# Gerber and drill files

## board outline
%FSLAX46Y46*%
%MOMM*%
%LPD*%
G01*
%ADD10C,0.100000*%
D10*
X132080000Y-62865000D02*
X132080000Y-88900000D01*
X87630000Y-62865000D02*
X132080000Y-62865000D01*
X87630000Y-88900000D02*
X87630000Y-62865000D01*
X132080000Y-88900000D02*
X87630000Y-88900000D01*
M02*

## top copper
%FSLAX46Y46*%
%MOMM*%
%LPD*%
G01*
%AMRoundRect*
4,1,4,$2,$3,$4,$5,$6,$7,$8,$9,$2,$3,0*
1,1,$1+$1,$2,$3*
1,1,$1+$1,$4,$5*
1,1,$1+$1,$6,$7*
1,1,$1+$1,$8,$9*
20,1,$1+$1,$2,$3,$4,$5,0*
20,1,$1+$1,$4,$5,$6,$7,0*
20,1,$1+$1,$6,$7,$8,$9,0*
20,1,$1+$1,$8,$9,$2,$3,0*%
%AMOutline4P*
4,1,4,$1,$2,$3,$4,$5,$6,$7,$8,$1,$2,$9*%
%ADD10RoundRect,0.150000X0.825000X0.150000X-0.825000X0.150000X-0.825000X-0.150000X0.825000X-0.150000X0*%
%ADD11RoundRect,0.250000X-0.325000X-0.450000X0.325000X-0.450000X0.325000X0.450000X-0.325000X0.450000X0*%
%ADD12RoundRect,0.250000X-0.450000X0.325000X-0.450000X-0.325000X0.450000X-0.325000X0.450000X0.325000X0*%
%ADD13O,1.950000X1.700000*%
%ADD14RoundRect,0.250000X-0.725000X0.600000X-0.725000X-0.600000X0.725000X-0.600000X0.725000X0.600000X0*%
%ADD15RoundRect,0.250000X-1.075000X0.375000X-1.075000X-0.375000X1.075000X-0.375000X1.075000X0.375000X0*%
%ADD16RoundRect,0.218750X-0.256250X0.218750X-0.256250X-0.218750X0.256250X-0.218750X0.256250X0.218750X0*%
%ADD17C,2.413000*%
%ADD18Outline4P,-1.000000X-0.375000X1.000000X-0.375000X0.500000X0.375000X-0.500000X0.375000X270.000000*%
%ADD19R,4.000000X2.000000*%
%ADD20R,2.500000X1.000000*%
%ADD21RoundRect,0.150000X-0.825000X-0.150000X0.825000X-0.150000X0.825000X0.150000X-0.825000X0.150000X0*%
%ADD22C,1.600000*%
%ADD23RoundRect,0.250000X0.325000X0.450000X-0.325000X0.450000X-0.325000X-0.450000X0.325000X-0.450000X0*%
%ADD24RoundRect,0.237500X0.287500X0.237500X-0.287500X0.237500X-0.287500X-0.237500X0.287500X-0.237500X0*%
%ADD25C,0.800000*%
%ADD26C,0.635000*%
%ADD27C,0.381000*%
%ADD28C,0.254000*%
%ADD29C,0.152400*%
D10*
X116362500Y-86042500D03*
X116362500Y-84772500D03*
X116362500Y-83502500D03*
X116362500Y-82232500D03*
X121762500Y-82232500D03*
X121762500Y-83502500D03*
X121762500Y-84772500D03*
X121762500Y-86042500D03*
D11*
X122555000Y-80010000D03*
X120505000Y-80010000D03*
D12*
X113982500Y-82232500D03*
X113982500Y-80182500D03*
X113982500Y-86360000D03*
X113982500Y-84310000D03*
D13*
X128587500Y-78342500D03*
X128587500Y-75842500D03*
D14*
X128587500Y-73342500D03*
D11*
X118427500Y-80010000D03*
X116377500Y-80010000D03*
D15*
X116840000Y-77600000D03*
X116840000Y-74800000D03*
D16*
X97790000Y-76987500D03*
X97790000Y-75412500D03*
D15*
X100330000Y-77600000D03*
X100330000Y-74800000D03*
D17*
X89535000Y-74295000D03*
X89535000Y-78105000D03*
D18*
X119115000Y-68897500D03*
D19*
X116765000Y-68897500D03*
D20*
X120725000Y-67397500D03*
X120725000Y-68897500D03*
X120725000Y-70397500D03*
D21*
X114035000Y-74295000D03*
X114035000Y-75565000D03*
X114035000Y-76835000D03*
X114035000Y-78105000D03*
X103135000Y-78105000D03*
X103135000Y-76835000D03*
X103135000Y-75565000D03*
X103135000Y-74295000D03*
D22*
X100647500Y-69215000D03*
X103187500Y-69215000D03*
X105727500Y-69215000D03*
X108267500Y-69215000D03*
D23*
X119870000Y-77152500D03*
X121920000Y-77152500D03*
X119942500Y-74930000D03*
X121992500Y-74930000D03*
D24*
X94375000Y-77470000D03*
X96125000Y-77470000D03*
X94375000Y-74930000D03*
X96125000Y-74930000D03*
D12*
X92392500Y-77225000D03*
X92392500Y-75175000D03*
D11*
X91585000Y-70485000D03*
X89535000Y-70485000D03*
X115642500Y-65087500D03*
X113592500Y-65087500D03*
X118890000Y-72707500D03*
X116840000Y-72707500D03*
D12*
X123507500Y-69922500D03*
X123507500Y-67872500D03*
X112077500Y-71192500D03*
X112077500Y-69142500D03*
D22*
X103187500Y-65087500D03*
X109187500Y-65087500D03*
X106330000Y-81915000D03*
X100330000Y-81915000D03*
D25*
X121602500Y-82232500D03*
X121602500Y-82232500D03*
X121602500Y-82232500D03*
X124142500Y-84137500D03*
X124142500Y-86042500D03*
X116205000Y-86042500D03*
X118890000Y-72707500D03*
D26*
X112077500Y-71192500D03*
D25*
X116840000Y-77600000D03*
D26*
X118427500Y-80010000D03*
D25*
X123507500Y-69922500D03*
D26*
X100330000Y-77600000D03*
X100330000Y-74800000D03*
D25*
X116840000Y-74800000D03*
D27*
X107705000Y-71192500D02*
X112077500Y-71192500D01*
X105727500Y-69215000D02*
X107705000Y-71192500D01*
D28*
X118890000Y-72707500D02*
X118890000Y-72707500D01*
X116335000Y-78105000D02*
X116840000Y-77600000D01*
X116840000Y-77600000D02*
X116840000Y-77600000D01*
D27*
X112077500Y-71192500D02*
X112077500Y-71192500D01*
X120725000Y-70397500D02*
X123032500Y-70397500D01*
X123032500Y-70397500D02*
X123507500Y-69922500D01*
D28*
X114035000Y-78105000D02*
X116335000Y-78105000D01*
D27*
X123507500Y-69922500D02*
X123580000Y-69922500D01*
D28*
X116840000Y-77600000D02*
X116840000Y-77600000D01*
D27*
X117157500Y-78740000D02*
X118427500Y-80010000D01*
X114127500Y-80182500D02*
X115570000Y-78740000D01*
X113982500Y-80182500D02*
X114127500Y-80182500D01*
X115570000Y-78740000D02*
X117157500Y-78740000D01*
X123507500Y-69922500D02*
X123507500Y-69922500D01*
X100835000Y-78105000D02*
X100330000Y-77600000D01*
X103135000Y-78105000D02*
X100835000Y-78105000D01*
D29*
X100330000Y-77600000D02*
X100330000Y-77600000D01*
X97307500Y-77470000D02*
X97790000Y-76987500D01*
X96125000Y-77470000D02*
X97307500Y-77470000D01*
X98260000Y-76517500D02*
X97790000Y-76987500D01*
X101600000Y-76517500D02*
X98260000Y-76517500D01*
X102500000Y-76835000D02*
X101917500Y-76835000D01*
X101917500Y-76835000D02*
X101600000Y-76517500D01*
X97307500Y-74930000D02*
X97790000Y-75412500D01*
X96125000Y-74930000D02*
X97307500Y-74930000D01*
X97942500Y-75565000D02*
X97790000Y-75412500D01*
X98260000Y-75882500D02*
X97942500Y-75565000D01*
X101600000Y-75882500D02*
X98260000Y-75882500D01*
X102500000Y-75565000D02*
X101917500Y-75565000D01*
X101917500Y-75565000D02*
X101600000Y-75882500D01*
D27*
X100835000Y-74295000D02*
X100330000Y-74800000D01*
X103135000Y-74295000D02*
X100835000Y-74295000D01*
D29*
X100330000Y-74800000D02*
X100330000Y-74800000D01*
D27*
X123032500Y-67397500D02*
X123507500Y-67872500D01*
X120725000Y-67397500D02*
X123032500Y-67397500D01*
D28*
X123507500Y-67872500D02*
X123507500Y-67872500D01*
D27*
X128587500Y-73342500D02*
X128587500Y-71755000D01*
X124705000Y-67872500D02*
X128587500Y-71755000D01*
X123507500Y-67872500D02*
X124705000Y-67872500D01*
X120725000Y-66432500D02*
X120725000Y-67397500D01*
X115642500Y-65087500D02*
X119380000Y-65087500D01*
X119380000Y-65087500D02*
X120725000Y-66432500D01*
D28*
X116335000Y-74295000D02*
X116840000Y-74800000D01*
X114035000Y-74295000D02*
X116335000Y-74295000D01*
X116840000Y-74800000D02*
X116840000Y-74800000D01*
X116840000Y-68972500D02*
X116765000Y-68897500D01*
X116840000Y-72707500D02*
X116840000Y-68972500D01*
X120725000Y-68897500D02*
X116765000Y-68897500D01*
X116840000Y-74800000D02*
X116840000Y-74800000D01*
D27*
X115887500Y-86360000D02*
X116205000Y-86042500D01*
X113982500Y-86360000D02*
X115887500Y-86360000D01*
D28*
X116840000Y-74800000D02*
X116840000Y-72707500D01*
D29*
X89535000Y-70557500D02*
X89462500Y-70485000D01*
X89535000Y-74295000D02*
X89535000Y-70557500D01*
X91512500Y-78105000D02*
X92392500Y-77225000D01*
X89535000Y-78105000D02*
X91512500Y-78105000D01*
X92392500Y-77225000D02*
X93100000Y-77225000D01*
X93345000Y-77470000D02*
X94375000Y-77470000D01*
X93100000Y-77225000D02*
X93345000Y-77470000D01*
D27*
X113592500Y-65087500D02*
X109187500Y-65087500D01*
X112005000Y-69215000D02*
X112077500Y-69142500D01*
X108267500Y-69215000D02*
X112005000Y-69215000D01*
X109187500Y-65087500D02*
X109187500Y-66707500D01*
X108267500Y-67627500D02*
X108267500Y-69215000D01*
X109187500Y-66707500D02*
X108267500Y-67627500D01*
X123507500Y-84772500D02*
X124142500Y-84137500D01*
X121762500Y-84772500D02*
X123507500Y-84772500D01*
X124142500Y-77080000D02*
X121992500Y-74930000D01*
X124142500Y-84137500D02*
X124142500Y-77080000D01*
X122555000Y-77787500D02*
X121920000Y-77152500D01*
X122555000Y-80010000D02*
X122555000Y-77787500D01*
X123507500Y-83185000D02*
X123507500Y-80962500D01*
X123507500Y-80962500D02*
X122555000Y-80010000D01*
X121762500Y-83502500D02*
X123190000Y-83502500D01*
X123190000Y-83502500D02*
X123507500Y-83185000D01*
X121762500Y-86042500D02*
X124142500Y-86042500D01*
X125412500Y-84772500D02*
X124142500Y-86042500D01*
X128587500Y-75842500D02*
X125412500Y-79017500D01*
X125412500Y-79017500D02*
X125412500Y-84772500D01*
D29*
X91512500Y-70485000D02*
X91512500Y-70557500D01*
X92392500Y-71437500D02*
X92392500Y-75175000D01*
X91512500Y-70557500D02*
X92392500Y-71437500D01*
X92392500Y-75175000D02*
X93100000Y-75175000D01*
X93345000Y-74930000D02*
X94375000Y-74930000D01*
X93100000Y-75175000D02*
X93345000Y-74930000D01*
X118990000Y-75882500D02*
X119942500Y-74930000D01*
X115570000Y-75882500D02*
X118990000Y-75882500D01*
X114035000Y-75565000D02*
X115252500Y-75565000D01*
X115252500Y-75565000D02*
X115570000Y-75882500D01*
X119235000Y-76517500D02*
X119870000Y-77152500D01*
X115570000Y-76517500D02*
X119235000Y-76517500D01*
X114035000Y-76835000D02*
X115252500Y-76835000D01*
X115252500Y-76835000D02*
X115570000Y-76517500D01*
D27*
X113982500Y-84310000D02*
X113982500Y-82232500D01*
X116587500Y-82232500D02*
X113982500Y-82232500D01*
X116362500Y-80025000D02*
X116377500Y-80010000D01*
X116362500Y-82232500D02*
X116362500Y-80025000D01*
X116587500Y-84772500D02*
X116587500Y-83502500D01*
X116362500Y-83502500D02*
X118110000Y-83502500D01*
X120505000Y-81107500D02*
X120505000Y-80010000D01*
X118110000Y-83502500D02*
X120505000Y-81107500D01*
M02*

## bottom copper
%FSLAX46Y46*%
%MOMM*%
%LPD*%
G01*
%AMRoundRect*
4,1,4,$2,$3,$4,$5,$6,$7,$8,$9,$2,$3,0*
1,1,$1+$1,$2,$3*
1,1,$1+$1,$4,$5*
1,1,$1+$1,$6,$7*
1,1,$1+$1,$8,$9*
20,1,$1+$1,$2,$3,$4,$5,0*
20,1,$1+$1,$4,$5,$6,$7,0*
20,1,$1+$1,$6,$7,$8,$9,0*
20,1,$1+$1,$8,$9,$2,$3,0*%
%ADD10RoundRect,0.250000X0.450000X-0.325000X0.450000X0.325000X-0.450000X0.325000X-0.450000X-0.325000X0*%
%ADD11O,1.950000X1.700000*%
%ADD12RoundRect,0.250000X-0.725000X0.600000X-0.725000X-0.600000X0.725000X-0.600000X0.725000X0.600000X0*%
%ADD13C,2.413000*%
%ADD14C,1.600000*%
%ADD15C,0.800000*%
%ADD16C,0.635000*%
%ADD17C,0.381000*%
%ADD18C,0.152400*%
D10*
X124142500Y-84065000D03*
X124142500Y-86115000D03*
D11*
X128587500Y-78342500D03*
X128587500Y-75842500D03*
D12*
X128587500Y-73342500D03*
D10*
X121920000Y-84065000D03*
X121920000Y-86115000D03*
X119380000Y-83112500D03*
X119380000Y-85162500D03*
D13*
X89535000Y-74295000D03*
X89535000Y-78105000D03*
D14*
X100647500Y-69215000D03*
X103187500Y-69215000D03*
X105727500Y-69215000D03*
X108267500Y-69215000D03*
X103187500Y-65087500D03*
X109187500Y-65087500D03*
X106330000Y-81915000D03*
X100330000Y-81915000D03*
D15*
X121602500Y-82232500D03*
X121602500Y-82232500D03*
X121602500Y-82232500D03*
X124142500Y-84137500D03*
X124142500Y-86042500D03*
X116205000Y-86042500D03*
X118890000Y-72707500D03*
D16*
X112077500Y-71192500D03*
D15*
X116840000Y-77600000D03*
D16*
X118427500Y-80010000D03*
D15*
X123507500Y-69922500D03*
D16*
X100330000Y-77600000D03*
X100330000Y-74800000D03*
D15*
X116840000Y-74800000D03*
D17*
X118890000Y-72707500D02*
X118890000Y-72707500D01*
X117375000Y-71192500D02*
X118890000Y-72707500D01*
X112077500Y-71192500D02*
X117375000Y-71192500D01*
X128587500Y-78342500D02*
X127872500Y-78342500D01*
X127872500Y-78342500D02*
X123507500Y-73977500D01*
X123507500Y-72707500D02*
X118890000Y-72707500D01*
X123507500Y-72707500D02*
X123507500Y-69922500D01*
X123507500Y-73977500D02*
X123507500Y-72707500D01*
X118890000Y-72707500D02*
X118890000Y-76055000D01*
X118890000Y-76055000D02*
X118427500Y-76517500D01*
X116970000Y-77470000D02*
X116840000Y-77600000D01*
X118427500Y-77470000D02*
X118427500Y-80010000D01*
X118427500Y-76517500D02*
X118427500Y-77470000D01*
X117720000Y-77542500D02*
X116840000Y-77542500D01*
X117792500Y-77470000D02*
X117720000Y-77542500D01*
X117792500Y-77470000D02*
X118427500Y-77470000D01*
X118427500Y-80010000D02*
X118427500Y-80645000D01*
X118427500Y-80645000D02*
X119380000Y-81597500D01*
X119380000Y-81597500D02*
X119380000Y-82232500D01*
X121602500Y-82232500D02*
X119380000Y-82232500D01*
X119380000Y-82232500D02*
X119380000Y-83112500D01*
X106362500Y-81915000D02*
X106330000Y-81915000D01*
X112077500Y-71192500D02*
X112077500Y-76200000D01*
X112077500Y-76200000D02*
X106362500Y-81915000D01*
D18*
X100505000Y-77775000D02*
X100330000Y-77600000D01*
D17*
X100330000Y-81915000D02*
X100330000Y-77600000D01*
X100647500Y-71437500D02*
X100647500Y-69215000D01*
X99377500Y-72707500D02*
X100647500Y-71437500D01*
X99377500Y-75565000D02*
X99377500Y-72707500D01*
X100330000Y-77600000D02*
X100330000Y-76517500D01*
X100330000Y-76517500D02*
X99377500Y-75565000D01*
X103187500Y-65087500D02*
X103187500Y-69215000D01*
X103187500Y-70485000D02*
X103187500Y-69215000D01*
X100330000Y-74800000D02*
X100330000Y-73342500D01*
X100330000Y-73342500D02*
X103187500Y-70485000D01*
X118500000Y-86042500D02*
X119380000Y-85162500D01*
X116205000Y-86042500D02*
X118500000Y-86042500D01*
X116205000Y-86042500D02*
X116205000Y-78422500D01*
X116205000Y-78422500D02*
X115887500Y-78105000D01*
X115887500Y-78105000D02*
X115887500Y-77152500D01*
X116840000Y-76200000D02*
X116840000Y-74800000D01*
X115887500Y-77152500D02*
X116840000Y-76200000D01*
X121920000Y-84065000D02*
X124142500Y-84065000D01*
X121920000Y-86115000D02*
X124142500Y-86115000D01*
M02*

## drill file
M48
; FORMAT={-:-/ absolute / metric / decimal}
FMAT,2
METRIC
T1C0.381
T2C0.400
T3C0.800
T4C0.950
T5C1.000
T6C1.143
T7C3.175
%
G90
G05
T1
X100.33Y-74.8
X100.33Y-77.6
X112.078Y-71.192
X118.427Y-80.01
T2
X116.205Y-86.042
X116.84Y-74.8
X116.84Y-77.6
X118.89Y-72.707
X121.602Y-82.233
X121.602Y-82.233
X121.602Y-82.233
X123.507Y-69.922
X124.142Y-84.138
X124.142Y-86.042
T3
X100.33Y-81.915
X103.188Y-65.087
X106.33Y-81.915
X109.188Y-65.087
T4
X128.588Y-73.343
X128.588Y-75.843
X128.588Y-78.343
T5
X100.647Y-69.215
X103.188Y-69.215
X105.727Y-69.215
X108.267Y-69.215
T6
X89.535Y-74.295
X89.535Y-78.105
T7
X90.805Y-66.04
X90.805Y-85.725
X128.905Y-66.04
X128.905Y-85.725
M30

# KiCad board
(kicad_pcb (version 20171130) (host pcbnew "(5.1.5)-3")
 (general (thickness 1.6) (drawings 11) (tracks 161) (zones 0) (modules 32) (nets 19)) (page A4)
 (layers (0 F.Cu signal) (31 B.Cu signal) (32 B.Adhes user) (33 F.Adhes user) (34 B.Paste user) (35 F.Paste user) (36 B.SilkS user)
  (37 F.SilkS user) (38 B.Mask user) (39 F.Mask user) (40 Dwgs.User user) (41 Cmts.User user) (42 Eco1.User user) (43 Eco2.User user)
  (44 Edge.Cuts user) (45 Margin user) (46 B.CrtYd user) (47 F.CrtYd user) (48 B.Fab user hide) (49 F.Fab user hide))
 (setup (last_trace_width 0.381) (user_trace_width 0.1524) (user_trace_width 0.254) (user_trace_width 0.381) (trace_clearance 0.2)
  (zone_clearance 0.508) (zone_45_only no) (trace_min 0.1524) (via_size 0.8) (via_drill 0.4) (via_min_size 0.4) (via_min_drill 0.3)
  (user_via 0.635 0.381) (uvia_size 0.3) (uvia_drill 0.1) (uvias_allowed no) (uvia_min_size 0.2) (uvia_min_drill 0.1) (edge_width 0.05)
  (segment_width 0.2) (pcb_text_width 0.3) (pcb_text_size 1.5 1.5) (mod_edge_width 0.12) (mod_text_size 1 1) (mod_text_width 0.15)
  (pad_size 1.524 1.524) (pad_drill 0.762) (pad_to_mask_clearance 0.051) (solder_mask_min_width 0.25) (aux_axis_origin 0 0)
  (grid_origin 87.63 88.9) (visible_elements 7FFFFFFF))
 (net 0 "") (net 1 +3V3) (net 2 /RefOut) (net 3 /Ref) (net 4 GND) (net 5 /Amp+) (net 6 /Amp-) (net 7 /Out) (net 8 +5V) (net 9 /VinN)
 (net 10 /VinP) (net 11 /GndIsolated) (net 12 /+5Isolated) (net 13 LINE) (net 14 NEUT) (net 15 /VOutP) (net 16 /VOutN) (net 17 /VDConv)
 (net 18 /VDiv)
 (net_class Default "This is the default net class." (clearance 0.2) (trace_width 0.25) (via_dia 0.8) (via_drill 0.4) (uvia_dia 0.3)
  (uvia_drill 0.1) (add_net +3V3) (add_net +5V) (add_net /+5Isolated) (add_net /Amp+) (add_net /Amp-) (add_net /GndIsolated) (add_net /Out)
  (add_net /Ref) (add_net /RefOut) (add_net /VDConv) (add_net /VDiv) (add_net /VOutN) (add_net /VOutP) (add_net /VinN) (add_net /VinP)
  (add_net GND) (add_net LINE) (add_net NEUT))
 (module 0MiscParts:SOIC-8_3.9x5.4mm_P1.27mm (layer F.Cu) (at 119.0625 84.1375 180)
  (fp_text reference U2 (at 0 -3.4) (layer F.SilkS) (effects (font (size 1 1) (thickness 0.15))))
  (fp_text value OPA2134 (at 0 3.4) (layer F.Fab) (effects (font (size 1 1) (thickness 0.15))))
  (pad 8 smd roundrect (at 2.7 -1.905 180) (size 1.95 0.6) (layers F.Cu F.Paste F.Mask) (roundrect_rratio 0.25) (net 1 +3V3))
  (pad 7 smd roundrect (at 2.7 -0.635 180) (size 1.95 0.6) (layers F.Cu F.Paste F.Mask) (roundrect_rratio 0.25) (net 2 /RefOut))
  (pad 6 smd roundrect (at 2.7 0.635 180) (size 1.95 0.6) (layers F.Cu F.Paste F.Mask) (roundrect_rratio 0.25) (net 2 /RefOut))
  (pad 5 smd roundrect (at 2.7 1.905 180) (size 1.95 0.6) (layers F.Cu F.Paste F.Mask) (roundrect_rratio 0.25) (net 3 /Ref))
  (pad 4 smd roundrect (at -2.7 1.905 180) (size 1.95 0.6) (layers F.Cu F.Paste F.Mask) (roundrect_rratio 0.25) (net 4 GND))
  (pad 3 smd roundrect (at -2.7 0.635 180) (size 1.95 0.6) (layers F.Cu F.Paste F.Mask) (roundrect_rratio 0.25) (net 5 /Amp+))
  (pad 2 smd roundrect (at -2.7 -0.635 180) (size 1.95 0.6) (layers F.Cu F.Paste F.Mask) (roundrect_rratio 0.25) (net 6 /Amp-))
  (pad 1 smd roundrect (at -2.7 -1.905 180) (size 1.95 0.6) (layers F.Cu F.Paste F.Mask) (roundrect_rratio 0.25) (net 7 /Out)))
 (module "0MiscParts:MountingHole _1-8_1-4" (layer F.Cu) (at 128.905 85.725)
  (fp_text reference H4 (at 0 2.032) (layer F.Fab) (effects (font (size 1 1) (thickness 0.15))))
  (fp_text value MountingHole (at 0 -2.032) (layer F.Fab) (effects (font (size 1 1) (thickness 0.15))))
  (pad "" np_thru_hole circle (at 0 0) (size 3.175 3.175) (drill 3.175) (layers *.Cu *.Mask)))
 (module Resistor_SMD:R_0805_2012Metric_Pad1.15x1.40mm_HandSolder (layer B.Cu) (at 124.1425 85.09 90)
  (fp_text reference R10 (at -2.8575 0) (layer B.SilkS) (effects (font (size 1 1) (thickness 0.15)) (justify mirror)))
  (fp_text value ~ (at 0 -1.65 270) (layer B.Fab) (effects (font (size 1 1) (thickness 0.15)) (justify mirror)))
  (pad 2 smd roundrect (at 1.025 0 90) (size 1.15 1.4) (layers B.Cu B.Paste B.Mask) (roundrect_rratio 0.217391) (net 6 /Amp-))
  (pad 1 smd roundrect (at -1.025 0 90) (size 1.15 1.4) (layers B.Cu B.Paste B.Mask) (roundrect_rratio 0.217391) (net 7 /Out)))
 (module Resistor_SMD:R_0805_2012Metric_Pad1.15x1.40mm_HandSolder (layer F.Cu) (at 121.53 80.01)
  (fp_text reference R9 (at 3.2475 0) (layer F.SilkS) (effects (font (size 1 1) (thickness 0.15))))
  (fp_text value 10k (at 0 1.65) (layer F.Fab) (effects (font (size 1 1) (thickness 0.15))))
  (pad 2 smd roundrect (at 1.025 0) (size 1.15 1.4) (layers F.Cu F.Paste F.Mask) (roundrect_rratio 0.217391) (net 5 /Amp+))
  (pad 1 smd roundrect (at -1.025 0) (size 1.15 1.4) (layers F.Cu F.Paste F.Mask) (roundrect_rratio 0.217391) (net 2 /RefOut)))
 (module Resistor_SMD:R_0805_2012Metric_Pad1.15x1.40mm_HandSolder (layer F.Cu) (at 113.9825 81.2075 270)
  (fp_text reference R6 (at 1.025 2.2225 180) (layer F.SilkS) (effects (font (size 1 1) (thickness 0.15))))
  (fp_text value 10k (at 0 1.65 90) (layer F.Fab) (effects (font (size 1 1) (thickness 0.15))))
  (pad 2 smd roundrect (at 1.025 0 270) (size 1.15 1.4) (layers F.Cu F.Paste F.Mask) (roundrect_rratio 0.217391) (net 3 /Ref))
  (pad 1 smd roundrect (at -1.025 0 270) (size 1.15 1.4) (layers F.Cu F.Paste F.Mask) (roundrect_rratio 0.217391) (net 4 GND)))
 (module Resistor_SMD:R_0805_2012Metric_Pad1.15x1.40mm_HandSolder (layer F.Cu) (at 113.9825 85.335 270)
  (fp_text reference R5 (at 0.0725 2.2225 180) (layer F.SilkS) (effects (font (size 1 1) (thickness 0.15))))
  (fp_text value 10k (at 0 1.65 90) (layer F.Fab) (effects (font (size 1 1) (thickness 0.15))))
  (pad 2 smd roundrect (at 1.025 0 270) (size 1.15 1.4) (layers F.Cu F.Paste F.Mask) (roundrect_rratio 0.217391) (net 1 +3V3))
  (pad 1 smd roundrect (at -1.025 0 270) (size 1.15 1.4) (layers F.Cu F.Paste F.Mask) (roundrect_rratio 0.217391) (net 3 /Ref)))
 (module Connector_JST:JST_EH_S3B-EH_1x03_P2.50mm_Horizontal (layer F.Cu) (at 128.5875 73.3425 270)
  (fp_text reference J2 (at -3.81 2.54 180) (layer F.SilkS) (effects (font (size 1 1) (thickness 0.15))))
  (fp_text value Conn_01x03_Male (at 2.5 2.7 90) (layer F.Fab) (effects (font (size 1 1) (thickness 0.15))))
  (pad 3 thru_hole oval (at 5 0 270) (size 1.7 1.95) (drill 0.95) (layers *.Cu *.Mask) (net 4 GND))
  (pad 2 thru_hole oval (at 2.5 0 270) (size 1.7 1.95) (drill 0.95) (layers *.Cu *.Mask) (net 7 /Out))
  (pad 1 thru_hole roundrect (at 0 0 270) (size 1.7 1.95) (drill 0.95) (layers *.Cu *.Mask) (roundrect_rratio 0.147059) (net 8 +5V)))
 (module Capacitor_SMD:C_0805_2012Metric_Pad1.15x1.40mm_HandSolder (layer B.Cu) (at 121.92 85.09 90)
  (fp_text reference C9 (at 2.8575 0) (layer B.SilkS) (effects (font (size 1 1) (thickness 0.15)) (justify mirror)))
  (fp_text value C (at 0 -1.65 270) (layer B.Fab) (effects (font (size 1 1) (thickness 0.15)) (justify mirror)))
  (pad 2 smd roundrect (at 1.025 0 90) (size 1.15 1.4) (layers B.Cu B.Paste B.Mask) (roundrect_rratio 0.217391) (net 6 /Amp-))
  (pad 1 smd roundrect (at -1.025 0 90) (size 1.15 1.4) (layers B.Cu B.Paste B.Mask) (roundrect_rratio 0.217391) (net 7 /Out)))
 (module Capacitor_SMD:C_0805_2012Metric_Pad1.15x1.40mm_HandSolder (layer B.Cu) (at 119.38 84.1375 90)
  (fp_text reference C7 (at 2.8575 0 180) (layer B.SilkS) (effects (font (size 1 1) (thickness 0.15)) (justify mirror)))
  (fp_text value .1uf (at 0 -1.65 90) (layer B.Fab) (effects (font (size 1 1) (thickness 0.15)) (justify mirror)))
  (pad 2 smd roundrect (at 1.025 0 90) (size 1.15 1.4) (layers B.Cu B.Paste B.Mask) (roundrect_rratio 0.217391) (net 4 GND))
  (pad 1 smd roundrect (at -1.025 0 90) (size 1.15 1.4) (layers B.Cu B.Paste B.Mask) (roundrect_rratio 0.217391) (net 1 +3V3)))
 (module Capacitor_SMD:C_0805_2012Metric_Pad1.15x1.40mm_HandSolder (layer F.Cu) (at 117.4025 80.01)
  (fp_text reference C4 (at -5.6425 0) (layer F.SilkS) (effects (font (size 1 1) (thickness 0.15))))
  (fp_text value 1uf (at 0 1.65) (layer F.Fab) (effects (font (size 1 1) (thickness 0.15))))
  (pad 2 smd roundrect (at 1.025 0) (size 1.15 1.4) (layers F.Cu F.Paste F.Mask) (roundrect_rratio 0.217391) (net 4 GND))
  (pad 1 smd roundrect (at -1.025 0) (size 1.15 1.4) (layers F.Cu F.Paste F.Mask) (roundrect_rratio 0.217391) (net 3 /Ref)))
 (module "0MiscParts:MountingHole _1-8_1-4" (layer F.Cu) (at 128.905 66.04)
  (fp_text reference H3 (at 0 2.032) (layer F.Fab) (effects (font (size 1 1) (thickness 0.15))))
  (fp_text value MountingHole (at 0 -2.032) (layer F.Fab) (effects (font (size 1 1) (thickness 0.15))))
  (pad "" np_thru_hole circle (at 0 0) (size 3.175 3.175) (drill 3.175) (layers *.Cu *.Mask)))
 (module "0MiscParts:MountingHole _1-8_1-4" (layer F.Cu) (at 90.805 85.725)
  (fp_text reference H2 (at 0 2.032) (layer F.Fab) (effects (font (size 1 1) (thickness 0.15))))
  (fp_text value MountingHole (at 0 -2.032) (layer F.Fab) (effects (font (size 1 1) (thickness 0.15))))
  (pad "" np_thru_hole circle (at 0 0) (size 3.175 3.175) (drill 3.175) (layers *.Cu *.Mask)))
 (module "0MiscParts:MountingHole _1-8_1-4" (layer F.Cu) (at 90.805 66.04)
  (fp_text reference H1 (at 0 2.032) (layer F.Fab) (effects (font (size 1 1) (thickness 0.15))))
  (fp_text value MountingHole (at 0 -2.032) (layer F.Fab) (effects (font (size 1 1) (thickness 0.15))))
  (pad "" np_thru_hole circle (at 0 0) (size 3.175 3.175) (drill 3.175) (layers *.Cu *.Mask)))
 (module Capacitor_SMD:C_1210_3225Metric (layer F.Cu) (at 116.84 76.2 270)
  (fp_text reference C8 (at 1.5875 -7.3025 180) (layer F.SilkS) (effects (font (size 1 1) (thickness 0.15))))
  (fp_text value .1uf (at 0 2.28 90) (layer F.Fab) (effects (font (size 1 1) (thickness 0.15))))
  (pad 2 smd roundrect (at 1.4 0 270) (size 1.25 2.65) (layers F.Cu F.Paste F.Mask) (roundrect_rratio 0.2) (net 4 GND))
  (pad 1 smd roundrect (at -1.4 0 270) (size 1.25 2.65) (layers F.Cu F.Paste F.Mask) (roundrect_rratio 0.2) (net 1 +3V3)))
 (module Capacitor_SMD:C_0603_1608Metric (layer F.Cu) (at 97.79 76.2 270)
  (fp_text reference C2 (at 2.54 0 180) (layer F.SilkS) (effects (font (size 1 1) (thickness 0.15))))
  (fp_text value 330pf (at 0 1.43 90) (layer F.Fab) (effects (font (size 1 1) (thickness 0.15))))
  (pad 2 smd roundrect (at 0.7875 0 270) (size 0.875 0.95) (layers F.Cu F.Paste F.Mask) (roundrect_rratio 0.25) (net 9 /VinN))
  (pad 1 smd roundrect (at -0.7875 0 270) (size 0.875 0.95) (layers F.Cu F.Paste F.Mask) (roundrect_rratio 0.25) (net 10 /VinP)))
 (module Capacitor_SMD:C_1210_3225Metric (layer F.Cu) (at 100.33 76.2 270)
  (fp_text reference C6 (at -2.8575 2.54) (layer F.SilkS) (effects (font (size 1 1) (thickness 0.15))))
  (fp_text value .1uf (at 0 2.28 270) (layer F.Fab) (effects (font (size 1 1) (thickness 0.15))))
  (pad 2 smd roundrect (at 1.4 0 270) (size 1.25 2.65) (layers F.Cu F.Paste F.Mask) (roundrect_rratio 0.2) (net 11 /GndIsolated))
  (pad 1 smd roundrect (at -1.4 0 270) (size 1.25 2.65) (layers F.Cu F.Paste F.Mask) (roundrect_rratio 0.2) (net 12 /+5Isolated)))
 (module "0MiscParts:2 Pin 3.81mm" (layer F.Cu) (at 89.535 76.2 270)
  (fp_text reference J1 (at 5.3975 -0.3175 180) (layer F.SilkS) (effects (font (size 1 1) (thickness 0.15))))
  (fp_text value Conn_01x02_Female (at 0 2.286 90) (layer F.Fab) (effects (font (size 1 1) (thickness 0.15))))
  (pad 1 thru_hole circle (at -1.905 0 270) (size 2.413 2.413) (drill 1.143) (layers *.Cu *.Mask) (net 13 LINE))
  (pad 2 thru_hole circle (at 1.905 0 270) (size 2.413 2.413) (drill 1.143) (layers *.Cu *.Mask) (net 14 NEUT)))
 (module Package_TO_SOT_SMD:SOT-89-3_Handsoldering (layer F.Cu) (at 118.745 68.8975 180)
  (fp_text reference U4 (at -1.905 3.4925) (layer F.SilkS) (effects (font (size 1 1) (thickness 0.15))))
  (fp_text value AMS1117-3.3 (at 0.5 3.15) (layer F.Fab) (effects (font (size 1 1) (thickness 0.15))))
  (pad 2 smd trapezoid (at -0.37 0 270) (size 1.5 0.75) (rect_delta 0 0.5) (layers F.Cu F.Paste F.Mask) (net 1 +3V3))
  (pad 2 smd rect (at 1.98 0 90) (size 2 4) (layers F.Cu F.Paste F.Mask) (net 1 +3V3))
  (pad 3 smd rect (at -1.98 1.5 90) (size 1 2.5) (layers F.Cu F.Paste F.Mask) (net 8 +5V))
  (pad 2 smd rect (at -1.98 0 90) (size 1 2.5) (layers F.Cu F.Paste F.Mask) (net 1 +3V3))
  (pad 1 smd rect (at -1.98 -1.5 90) (size 1 2.5) (layers F.Cu F.Paste F.Mask) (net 4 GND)))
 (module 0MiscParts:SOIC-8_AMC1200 (layer F.Cu) (at 108.585 76.2)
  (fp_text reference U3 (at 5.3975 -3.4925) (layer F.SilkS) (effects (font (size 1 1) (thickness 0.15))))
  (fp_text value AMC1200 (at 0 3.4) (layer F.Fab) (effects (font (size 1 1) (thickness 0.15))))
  (pad 8 smd roundrect (at 5.45 -1.905) (size 1.95 0.6) (layers F.Cu F.Paste F.Mask) (roundrect_rratio 0.25) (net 1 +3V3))
  (pad 7 smd roundrect (at 5.45 -0.635) (size 1.95 0.6) (layers F.Cu F.Paste F.Mask) (roundrect_rratio 0.25) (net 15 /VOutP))
  (pad 6 smd roundrect (at 5.45 0.635) (size 1.95 0.6) (layers F.Cu F.Paste F.Mask) (roundrect_rratio 0.25) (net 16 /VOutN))
  (pad 5 smd roundrect (at 5.45 1.905) (size 1.95 0.6) (layers F.Cu F.Paste F.Mask) (roundrect_rratio 0.25) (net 4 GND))
  (pad 4 smd roundrect (at -5.45 1.905) (size 1.95 0.6) (layers F.Cu F.Paste F.Mask) (roundrect_rratio 0.25) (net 11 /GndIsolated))
  (pad 3 smd roundrect (at -5.45 0.635) (size 1.95 0.6) (layers F.Cu F.Paste F.Mask) (roundrect_rratio 0.25) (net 9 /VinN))
  (pad 2 smd roundrect (at -5.45 -0.635) (size 1.95 0.6) (layers F.Cu F.Paste F.Mask) (roundrect_rratio 0.25) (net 10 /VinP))
  (pad 1 smd roundrect (at -5.45 -1.905) (size 1.95 0.6) (layers F.Cu F.Paste F.Mask) (roundrect_rratio 0.25) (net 12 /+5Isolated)))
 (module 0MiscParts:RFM (layer F.Cu) (at 104.4575 69.215 180)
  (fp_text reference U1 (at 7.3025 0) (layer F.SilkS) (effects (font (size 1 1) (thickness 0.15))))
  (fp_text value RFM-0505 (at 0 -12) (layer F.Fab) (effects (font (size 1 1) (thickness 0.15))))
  (pad 4 thru_hole circle (at 3.81 0 180) (size 1.6 1.6) (drill 1) (layers *.Cu *.Mask) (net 11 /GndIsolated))
  (pad 3 thru_hole circle (at 1.27 0 180) (size 1.6 1.6) (drill 1) (layers *.Cu *.Mask) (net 12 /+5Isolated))
  (pad 2 thru_hole circle (at -1.27 0 180) (size 1.6 1.6) (drill 1) (layers *.Cu *.Mask) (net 4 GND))
  (pad 1 thru_hole circle (at -3.81 0 180) (size 1.6 1.6) (drill 1) (layers *.Cu *.Mask) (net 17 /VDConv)))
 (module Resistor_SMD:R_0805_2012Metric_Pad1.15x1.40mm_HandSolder (layer F.Cu) (at 120.895 77.1525 180)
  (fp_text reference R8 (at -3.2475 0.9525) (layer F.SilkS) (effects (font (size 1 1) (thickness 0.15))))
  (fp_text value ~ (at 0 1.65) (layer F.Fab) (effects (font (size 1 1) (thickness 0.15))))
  (pad 2 smd roundrect (at 1.025 0 180) (size 1.15 1.4) (layers F.Cu F.Paste F.Mask) (roundrect_rratio 0.217391) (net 16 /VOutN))
  (pad 1 smd roundrect (at -1.025 0 180) (size 1.15 1.4) (layers F.Cu F.Paste F.Mask) (roundrect_rratio 0.217391) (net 5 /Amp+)))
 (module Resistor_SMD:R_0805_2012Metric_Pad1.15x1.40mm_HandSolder (layer F.Cu) (at 120.9675 74.93 180)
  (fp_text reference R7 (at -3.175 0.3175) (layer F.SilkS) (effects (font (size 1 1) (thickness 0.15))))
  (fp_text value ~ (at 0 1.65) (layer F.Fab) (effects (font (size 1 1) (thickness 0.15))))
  (pad 2 smd roundrect (at 1.025 0 180) (size 1.15 1.4) (layers F.Cu F.Paste F.Mask) (roundrect_rratio 0.217391) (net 15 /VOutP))
  (pad 1 smd roundrect (at -1.025 0 180) (size 1.15 1.4) (layers F.Cu F.Paste F.Mask) (roundrect_rratio 0.217391) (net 6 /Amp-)))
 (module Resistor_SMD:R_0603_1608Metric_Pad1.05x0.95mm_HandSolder (layer F.Cu) (at 95.25 77.47 180)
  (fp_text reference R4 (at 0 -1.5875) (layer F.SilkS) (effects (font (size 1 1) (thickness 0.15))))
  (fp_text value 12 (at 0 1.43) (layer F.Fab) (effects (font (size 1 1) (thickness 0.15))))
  (pad 2 smd roundrect (at 0.875 0 180) (size 1.05 0.95) (layers F.Cu F.Paste F.Mask) (roundrect_rratio 0.25) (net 14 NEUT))
  (pad 1 smd roundrect (at -0.875 0 180) (size 1.05 0.95) (layers F.Cu F.Paste F.Mask) (roundrect_rratio 0.25) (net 9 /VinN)))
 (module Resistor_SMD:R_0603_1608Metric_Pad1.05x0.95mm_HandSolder (layer F.Cu) (at 95.25 74.93 180)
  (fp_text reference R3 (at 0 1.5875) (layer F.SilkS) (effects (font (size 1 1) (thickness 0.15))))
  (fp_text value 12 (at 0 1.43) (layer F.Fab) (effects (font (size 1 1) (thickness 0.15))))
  (pad 2 smd roundrect (at 0.875 0 180) (size 1.05 0.95) (layers F.Cu F.Paste F.Mask) (roundrect_rratio 0.25) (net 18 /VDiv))
  (pad 1 smd roundrect (at -0.875 0 180) (size 1.05 0.95) (layers F.Cu F.Paste F.Mask) (roundrect_rratio 0.25) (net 10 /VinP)))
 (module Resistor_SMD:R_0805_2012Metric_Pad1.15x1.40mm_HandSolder (layer F.Cu) (at 92.3925 76.2 270)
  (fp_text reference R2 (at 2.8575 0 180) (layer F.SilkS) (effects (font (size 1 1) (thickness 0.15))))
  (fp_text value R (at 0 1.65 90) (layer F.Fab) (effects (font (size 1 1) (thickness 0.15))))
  (pad 2 smd roundrect (at 1.025 0 270) (size 1.15 1.4) (layers F.Cu F.Paste F.Mask) (roundrect_rratio 0.217391) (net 14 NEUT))
  (pad 1 smd roundrect (at -1.025 0 270) (size 1.15 1.4) (layers F.Cu F.Paste F.Mask) (roundrect_rratio 0.217391) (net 18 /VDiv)))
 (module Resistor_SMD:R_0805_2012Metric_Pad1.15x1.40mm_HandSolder (layer F.Cu) (at 90.56 70.485)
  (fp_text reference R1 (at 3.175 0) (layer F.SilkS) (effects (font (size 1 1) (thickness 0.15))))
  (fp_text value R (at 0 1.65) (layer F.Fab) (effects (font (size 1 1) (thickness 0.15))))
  (pad 2 smd roundrect (at 1.025 0) (size 1.15 1.4) (layers F.Cu F.Paste F.Mask) (roundrect_rratio 0.217391) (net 18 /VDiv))
  (pad 1 smd roundrect (at -1.025 0) (size 1.15 1.4) (layers F.Cu F.Paste F.Mask) (roundrect_rratio 0.217391) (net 13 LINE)))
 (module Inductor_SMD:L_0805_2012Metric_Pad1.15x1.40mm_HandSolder (layer F.Cu) (at 114.6175 65.0875)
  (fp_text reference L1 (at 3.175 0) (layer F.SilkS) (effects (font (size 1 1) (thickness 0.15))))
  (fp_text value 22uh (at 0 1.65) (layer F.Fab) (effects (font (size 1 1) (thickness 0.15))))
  (pad 2 smd roundrect (at 1.025 0) (size 1.15 1.4) (layers F.Cu F.Paste F.Mask) (roundrect_rratio 0.217391) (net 8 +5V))
  (pad 1 smd roundrect (at -1.025 0) (size 1.15 1.4) (layers F.Cu F.Paste F.Mask) (roundrect_rratio 0.217391) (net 17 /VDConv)))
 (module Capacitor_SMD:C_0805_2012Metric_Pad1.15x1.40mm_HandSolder (layer F.Cu) (at 117.865 72.7075)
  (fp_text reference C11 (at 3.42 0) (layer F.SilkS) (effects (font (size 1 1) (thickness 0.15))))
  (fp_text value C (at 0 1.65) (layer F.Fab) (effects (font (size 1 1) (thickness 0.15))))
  (pad 2 smd roundrect (at 1.025 0) (size 1.15 1.4) (layers F.Cu F.Paste F.Mask) (roundrect_rratio 0.217391) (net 4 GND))
  (pad 1 smd roundrect (at -1.025 0) (size 1.15 1.4) (layers F.Cu F.Paste F.Mask) (roundrect_rratio 0.217391) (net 1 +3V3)))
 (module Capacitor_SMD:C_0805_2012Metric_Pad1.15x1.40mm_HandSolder (layer F.Cu) (at 123.5075 68.8975 270)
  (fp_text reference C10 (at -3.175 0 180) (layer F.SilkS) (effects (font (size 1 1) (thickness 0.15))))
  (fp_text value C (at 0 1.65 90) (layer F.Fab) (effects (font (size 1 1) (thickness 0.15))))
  (pad 2 smd roundrect (at 1.025 0 270) (size 1.15 1.4) (layers F.Cu F.Paste F.Mask) (roundrect_rratio 0.217391) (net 4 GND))
  (pad 1 smd roundrect (at -1.025 0 270) (size 1.15 1.4) (layers F.Cu F.Paste F.Mask) (roundrect_rratio 0.217391) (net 8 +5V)))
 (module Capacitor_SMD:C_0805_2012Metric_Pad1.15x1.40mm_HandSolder (layer F.Cu) (at 112.0775 70.1675 270)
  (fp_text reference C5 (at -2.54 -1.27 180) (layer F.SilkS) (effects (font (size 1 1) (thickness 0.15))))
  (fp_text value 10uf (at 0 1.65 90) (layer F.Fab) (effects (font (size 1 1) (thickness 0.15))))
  (pad 2 smd roundrect (at 1.025 0 270) (size 1.15 1.4) (layers F.Cu F.Paste F.Mask) (roundrect_rratio 0.217391) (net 4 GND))
  (pad 1 smd roundrect (at -1.025 0 270) (size 1.15 1.4) (layers F.Cu F.Paste F.Mask) (roundrect_rratio 0.217391) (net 17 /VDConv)))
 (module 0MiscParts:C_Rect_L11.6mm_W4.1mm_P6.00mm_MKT (layer F.Cu) (at 106.1875 65.0875 180)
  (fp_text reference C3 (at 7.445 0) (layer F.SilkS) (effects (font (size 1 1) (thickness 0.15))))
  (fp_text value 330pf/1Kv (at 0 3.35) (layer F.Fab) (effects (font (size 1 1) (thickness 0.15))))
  (pad 2 thru_hole circle (at 3 0 180) (size 1.6 1.6) (drill 0.8) (layers *.Cu *.Mask) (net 12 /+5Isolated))
  (pad 1 thru_hole circle (at -3 0 180) (size 1.6 1.6) (drill 0.8) (layers *.Cu *.Mask) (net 17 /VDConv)))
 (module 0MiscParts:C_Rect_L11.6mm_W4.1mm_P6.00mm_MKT (layer F.Cu) (at 103.33 81.915)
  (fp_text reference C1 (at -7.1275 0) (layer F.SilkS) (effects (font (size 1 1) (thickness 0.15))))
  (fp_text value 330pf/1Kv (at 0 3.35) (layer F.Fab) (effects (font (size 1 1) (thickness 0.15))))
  (pad 2 thru_hole circle (at 3 0) (size 1.6 1.6) (drill 0.8) (layers *.Cu *.Mask) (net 4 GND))
  (pad 1 thru_hole circle (at -3 0) (size 1.6 1.6) (drill 0.8) (layers *.Cu *.Mask) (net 11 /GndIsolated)))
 (gr_line (start 132.08 62.865) (end 132.08 88.9) (layer Edge.Cuts) (width 0.1))
 (gr_line (start 87.63 62.865) (end 132.08 62.865) (layer Edge.Cuts) (width 0.1))
 (gr_line (start 87.63 88.9) (end 87.63 62.865) (layer Edge.Cuts) (width 0.1))
 (gr_line (start 132.08 88.9) (end 87.63 88.9) (layer Edge.Cuts) (width 0.1))
 (via (at 121.6025 82.2325) (size 0.8) (drill 0.4) (layers F.Cu B.Cu) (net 4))
 (via (at 121.6025 82.2325) (size 0.8) (drill 0.4) (layers F.Cu B.Cu) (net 4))
 (via (at 121.6025 82.2325) (size 0.8) (drill 0.4) (layers F.Cu B.Cu) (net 4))
 (via (at 124.1425 84.1375) (size 0.8) (drill 0.4) (layers F.Cu B.Cu) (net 6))
 (via (at 124.1425 86.0425) (size 0.8) (drill 0.4) (layers F.Cu B.Cu) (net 7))
 (via (at 116.205 86.0425) (size 0.8) (drill 0.4) (layers F.Cu B.Cu) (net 1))
 (segment (start 107.705 71.1925) (end 112.0775 71.1925) (width 0.381) (layer F.Cu) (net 4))
 (segment (start 105.7275 69.215) (end 107.705 71.1925) (width 0.381) (layer F.Cu) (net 4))
 (via (at 118.89 72.7075) (size 0.8) (drill 0.4) (layers F.Cu B.Cu) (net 4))
 (via (at 112.0775 71.1925) (size 0.635) (drill 0.381) (layers F.Cu B.Cu) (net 4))
 (via (at 116.84 77.6) (size 0.8) (drill 0.4) (layers F.Cu B.Cu) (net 4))
 (segment (start 118.89 72.7075) (end 118.89 72.7075) (width 0.254) (layer F.Cu) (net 4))
 (segment (start 116.335 78.105) (end 116.84 77.6) (width 0.254) (layer F.Cu) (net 4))
 (segment (start 116.84 77.6) (end 116.84 77.6) (width 0.254) (layer F.Cu) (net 4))
 (segment (start 112.0775 71.1925) (end 112.0775 71.1925) (width 0.381) (layer F.Cu) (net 4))
 (segment (start 120.725 70.3975) (end 123.0325 70.3975) (width 0.381) (layer F.Cu) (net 4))
 (segment (start 123.0325 70.3975) (end 123.5075 69.9225) (width 0.381) (layer F.Cu) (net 4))
 (segment (start 114.035 78.105) (end 116.335 78.105) (width 0.254) (layer F.Cu) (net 4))
 (segment (start 123.5075 69.9225) (end 123.58 69.9225) (width 0.381) (layer F.Cu) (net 4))
 (segment (start 116.84 77.6) (end 116.84 77.6) (width 0.254) (layer F.Cu) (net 4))
 (segment (start 118.89 72.7075) (end 118.89 72.7075) (width 0.381) (layer B.Cu) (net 4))
 (segment (start 117.375 71.1925) (end 118.89 72.7075) (width 0.381) (layer B.Cu) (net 4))
 (segment (start 112.0775 71.1925) (end 117.375 71.1925) (width 0.381) (layer B.Cu) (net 4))
 (segment (start 117.1575 78.74) (end 118.4275 80.01) (width 0.381) (layer F.Cu) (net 4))
 (via (at 118.4275 80.01) (size 0.635) (drill 0.381) (layers F.Cu B.Cu) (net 4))
 (segment (start 114.1275 80.1825) (end 115.57 78.74) (width 0.381) (layer F.Cu) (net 4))
 (segment (start 113.9825 80.1825) (end 114.1275 80.1825) (width 0.381) (layer F.Cu) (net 4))
 (segment (start 115.57 78.74) (end 117.1575 78.74) (width 0.381) (layer F.Cu) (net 4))
 (segment (start 123.5075 69.9225) (end 123.5075 69.9225) (width 0.381) (layer F.Cu) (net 4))
 (via (at 123.5075 69.9225) (size 0.8) (drill 0.4) (layers F.Cu B.Cu) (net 4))
 (segment (start 128.5875 78.3425) (end 127.8725 78.3425) (width 0.381) (layer B.Cu) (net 4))
 (segment (start 127.8725 78.3425) (end 123.5075 73.9775) (width 0.381) (layer B.Cu) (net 4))
 (segment (start 123.5075 72.7075) (end 118.89 72.7075) (width 0.381) (layer B.Cu) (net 4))
 (segment (start 123.5075 72.7075) (end 123.5075 69.9225) (width 0.381) (layer B.Cu) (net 4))
 (segment (start 123.5075 73.9775) (end 123.5075 72.7075) (width 0.381) (layer B.Cu) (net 4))
 (segment (start 118.89 72.7075) (end 118.89 76.055) (width 0.381) (layer B.Cu) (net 4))
 (segment (start 118.89 76.055) (end 118.4275 76.5175) (width 0.381) (layer B.Cu) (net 4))
 (segment (start 116.97 77.47) (end 116.84 77.6) (width 0.381) (layer B.Cu) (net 4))
 (segment (start 118.4275 77.47) (end 118.4275 80.01) (width 0.381) (layer B.Cu) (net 4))
 (segment (start 118.4275 76.5175) (end 118.4275 77.47) (width 0.381) (layer B.Cu) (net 4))
 (segment (start 117.72 77.5425) (end 116.84 77.5425) (width 0.381) (layer B.Cu) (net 4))
 (segment (start 117.7925 77.47) (end 117.72 77.5425) (width 0.381) (layer B.Cu) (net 4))
 (segment (start 117.7925 77.47) (end 118.4275 77.47) (width 0.381) (layer B.Cu) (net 4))
 (segment (start 118.4275 80.01) (end 118.4275 80.645) (width 0.381) (layer B.Cu) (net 4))
 (segment (start 118.4275 80.645) (end 119.38 81.5975) (width 0.381) (layer B.Cu) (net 4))
 (segment (start 119.38 81.5975) (end 119.38 82.2325) (width 0.381) (layer B.Cu) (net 4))
 (segment (start 121.6025 82.2325) (end 119.38 82.2325) (width 0.381) (layer B.Cu) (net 4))
 (segment (start 119.38 82.2325) (end 119.38 83.1125) (width 0.381) (layer B.Cu) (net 4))
 (segment (start 106.3625 81.915) (end 106.33 81.915) (width 0.381) (layer B.Cu) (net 4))
 (segment (start 112.0775 71.1925) (end 112.0775 76.2) (width 0.381) (layer B.Cu) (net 4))
 (segment (start 112.0775 76.2) (end 106.3625 81.915) (width 0.381) (layer B.Cu) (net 4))
 (segment (start 100.835 78.105) (end 100.33 77.6) (width 0.381) (layer F.Cu) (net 11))
 (segment (start 103.135 78.105) (end 100.835 78.105) (width 0.381) (layer F.Cu) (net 11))
 (segment (start 100.33 77.6) (end 100.33 77.6) (width 0.1524) (layer F.Cu) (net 11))
 (via (at 100.33 77.6) (size 0.635) (drill 0.381) (layers F.Cu B.Cu) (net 11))
 (segment (start 100.505 77.775) (end 100.33 77.6) (width 0.1524) (layer B.Cu) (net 11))
 (segment (start 100.33 81.915) (end 100.33 77.6) (width 0.381) (layer B.Cu) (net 11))
 (segment (start 100.6475 71.4375) (end 100.6475 69.215) (width 0.381) (layer B.Cu) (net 11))
 (segment (start 99.3775 72.7075) (end 100.6475 71.4375) (width 0.381) (layer B.Cu) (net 11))
 (segment (start 99.3775 75.565) (end 99.3775 72.7075) (width 0.381) (layer B.Cu) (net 11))
 (segment (start 100.33 77.6) (end 100.33 76.5175) (width 0.381) (layer B.Cu) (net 11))
 (segment (start 100.33 76.5175) (end 99.3775 75.565) (width 0.381) (layer B.Cu) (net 11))
 (segment (start 97.3075 77.47) (end 97.79 76.9875) (width 0.1524) (layer F.Cu) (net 9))
 (segment (start 96.125 77.47) (end 97.3075 77.47) (width 0.1524) (layer F.Cu) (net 9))
 (segment (start 98.26 76.5175) (end 97.79 76.9875) (width 0.1524) (layer F.Cu) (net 9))
 (segment (start 101.6 76.5175) (end 98.26 76.5175) (width 0.1524) (layer F.Cu) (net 9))
 (segment (start 102.5 76.835) (end 101.9175 76.835) (width 0.1524) (layer F.Cu) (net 9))
 (segment (start 101.9175 76.835) (end 101.6 76.5175) (width 0.1524) (layer F.Cu) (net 9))
 (segment (start 97.3075 74.93) (end 97.79 75.4125) (width 0.1524) (layer F.Cu) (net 10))
 (segment (start 96.125 74.93) (end 97.3075 74.93) (width 0.1524) (layer F.Cu) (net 10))
 (segment (start 97.9425 75.565) (end 97.79 75.4125) (width 0.1524) (layer F.Cu) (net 10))
 (segment (start 98.26 75.8825) (end 97.9425 75.565) (width 0.1524) (layer F.Cu) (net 10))
 (segment (start 101.6 75.8825) (end 98.26 75.8825) (width 0.1524) (layer F.Cu) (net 10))
 (segment (start 102.5 75.565) (end 101.9175 75.565) (width 0.1524) (layer F.Cu) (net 10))
 (segment (start 101.9175 75.565) (end 101.6 75.8825) (width 0.1524) (layer F.Cu) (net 10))
 (segment (start 100.835 74.295) (end 100.33 74.8) (width 0.381) (layer F.Cu) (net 12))
 (segment (start 103.135 74.295) (end 100.835 74.295) (width 0.381) (layer F.Cu) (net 12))
 (segment (start 100.33 74.8) (end 100.33 74.8) (width 0.1524) (layer F.Cu) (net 12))
 (via (at 100.33 74.8) (size 0.635) (drill 0.381) (layers F.Cu B.Cu) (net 12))
 (segment (start 103.1875 65.0875) (end 103.1875 69.215) (width 0.381) (layer B.Cu) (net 12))
 (segment (start 103.1875 70.485) (end 103.1875 69.215) (width 0.381) (layer B.Cu) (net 12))
 (segment (start 100.33 74.8) (end 100.33 73.3425) (width 0.381) (layer B.Cu) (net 12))
 (segment (start 100.33 73.3425) (end 103.1875 70.485) (width 0.381) (layer B.Cu) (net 12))
 (segment (start 123.0325 67.3975) (end 123.5075 67.8725) (width 0.381) (layer F.Cu) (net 8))
 (segment (start 120.725 67.3975) (end 123.0325 67.3975) (width 0.381) (layer F.Cu) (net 8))
 (segment (start 123.5075 67.8725) (end 123.5075 67.8725) (width 0.254) (layer F.Cu) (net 8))
 (segment (start 128.5875 73.3425) (end 128.5875 71.755) (width 0.381) (layer F.Cu) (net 8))
 (segment (start 124.705 67.8725) (end 128.5875 71.755) (width 0.381) (layer F.Cu) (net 8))
 (segment (start 123.5075 67.8725) (end 124.705 67.8725) (width 0.381) (layer F.Cu) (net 8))
 (segment (start 120.725 66.4325) (end 120.725 67.3975) (width 0.381) (layer F.Cu) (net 8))
 (segment (start 115.6425 65.0875) (end 119.38 65.0875) (width 0.381) (layer F.Cu) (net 8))
 (segment (start 119.38 65.0875) (end 120.725 66.4325) (width 0.381) (layer F.Cu) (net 8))
 (segment (start 116.335 74.295) (end 116.84 74.8) (width 0.254) (layer F.Cu) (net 1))
 (segment (start 114.035 74.295) (end 116.335 74.295) (width 0.254) (layer F.Cu) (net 1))
 (segment (start 116.84 74.8) (end 116.84 74.8) (width 0.254) (layer F.Cu) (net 1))
 (segment (start 116.84 68.9725) (end 116.765 68.8975) (width 0.254) (layer F.Cu) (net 1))
 (segment (start 116.84 72.7075) (end 116.84 68.9725) (width 0.254) (layer F.Cu) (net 1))
 (segment (start 120.725 68.8975) (end 116.765 68.8975) (width 0.254) (layer F.Cu) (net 1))
 (segment (start 116.84 74.8) (end 116.84 74.8) (width 0.254) (layer F.Cu) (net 1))
 (segment (start 115.8875 86.36) (end 116.205 86.0425) (width 0.381) (layer F.Cu) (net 1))
 (segment (start 113.9825 86.36) (end 115.8875 86.36) (width 0.381) (layer F.Cu) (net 1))
 (segment (start 118.5 86.0425) (end 119.38 85.1625) (width 0.381) (layer B.Cu) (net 1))
 (segment (start 116.205 86.0425) (end 118.5 86.0425) (width 0.381) (layer B.Cu) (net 1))
 (segment (start 116.84 74.8) (end 116.84 72.7075) (width 0.254) (layer F.Cu) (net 1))
 (via (at 116.84 74.8) (size 0.8) (drill 0.4) (layers F.Cu B.Cu) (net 1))
 (segment (start 116.205 86.0425) (end 116.205 78.4225) (width 0.381) (layer B.Cu) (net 1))
 (segment (start 116.205 78.4225) (end 115.8875 78.105) (width 0.381) (layer B.Cu) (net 1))
 (segment (start 115.8875 78.105) (end 115.8875 77.1525) (width 0.381) (layer B.Cu) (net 1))
 (segment (start 116.84 76.2) (end 116.84 74.8) (width 0.381) (layer B.Cu) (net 1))
 (segment (start 115.8875 77.1525) (end 116.84 76.2) (width 0.381) (layer B.Cu) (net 1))
 (segment (start 89.535 70.5575) (end 89.4625 70.485) (width 0.1524) (layer F.Cu) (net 13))
 (segment (start 89.535 74.295) (end 89.535 70.5575) (width 0.1524) (layer F.Cu) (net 13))
 (segment (start 91.5125 78.105) (end 92.3925 77.225) (width 0.1524) (layer F.Cu) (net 14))
 (segment (start 89.535 78.105) (end 91.5125 78.105) (width 0.1524) (layer F.Cu) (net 14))
 (segment (start 92.3925 77.225) (end 93.1 77.225) (width 0.1524) (layer F.Cu) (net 14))
 (segment (start 93.345 77.47) (end 94.375 77.47) (width 0.1524) (layer F.Cu) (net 14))
 (segment (start 93.1 77.225) (end 93.345 77.47) (width 0.1524) (layer F.Cu) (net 14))
 (segment (start 113.5925 65.0875) (end 109.1875 65.0875) (width 0.381) (layer F.Cu) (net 17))
 (segment (start 112.005 69.215) (end 112.0775 69.1425) (width 0.381) (layer F.Cu) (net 17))
 (segment (start 108.2675 69.215) (end 112.005 69.215) (width 0.381) (layer F.Cu) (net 17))
 (segment (start 109.1875 65.0875) (end 109.1875 66.7075) (width 0.381) (layer F.Cu) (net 17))
 (segment (start 108.2675 67.6275) (end 108.2675 69.215) (width 0.381) (layer F.Cu) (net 17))
 (segment (start 109.1875 66.7075) (end 108.2675 67.6275) (width 0.381) (layer F.Cu) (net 17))
 (segment (start 123.5075 84.7725) (end 124.1425 84.1375) (width 0.381) (layer F.Cu) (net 6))
 (segment (start 121.7625 84.7725) (end 123.5075 84.7725) (width 0.381) (layer F.Cu) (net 6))
 (segment (start 121.92 84.065) (end 124.1425 84.065) (width 0.381) (layer B.Cu) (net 6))
 (segment (start 124.1425 77.08) (end 121.9925 74.93) (width 0.381) (layer F.Cu) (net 6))
 (segment (start 124.1425 84.1375) (end 124.1425 77.08) (width 0.381) (layer F.Cu) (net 6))
 (segment (start 122.555 77.7875) (end 121.92 77.1525) (width 0.381) (layer F.Cu) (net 5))
 (segment (start 122.555 80.01) (end 122.555 77.7875) (width 0.381) (layer F.Cu) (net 5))
 (segment (start 123.5075 83.185) (end 123.5075 80.9625) (width 0.381) (layer F.Cu) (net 5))
 (segment (start 123.5075 80.9625) (end 122.555 80.01) (width 0.381) (layer F.Cu) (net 5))
 (segment (start 121.7625 83.5025) (end 123.19 83.5025) (width 0.381) (layer F.Cu) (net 5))
 (segment (start 123.19 83.5025) (end 123.5075 83.185) (width 0.381) (layer F.Cu) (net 5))
 (segment (start 121.7625 86.0425) (end 124.1425 86.0425) (width 0.381) (layer F.Cu) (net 7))
 (segment (start 121.92 86.115) (end 124.1425 86.115) (width 0.381) (layer B.Cu) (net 7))
 (segment (start 125.4125 84.7725) (end 124.1425 86.0425) (width 0.381) (layer F.Cu) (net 7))
 (segment (start 128.5875 75.8425) (end 125.4125 79.0175) (width 0.381) (layer F.Cu) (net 7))
 (segment (start 125.4125 79.0175) (end 125.4125 84.7725) (width 0.381) (layer F.Cu) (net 7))
 (segment (start 91.5125 70.485) (end 91.5125 70.5575) (width 0.1524) (layer F.Cu) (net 18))
 (segment (start 92.3925 71.4375) (end 92.3925 75.175) (width 0.1524) (layer F.Cu) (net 18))
 (segment (start 91.5125 70.5575) (end 92.3925 71.4375) (width 0.1524) (layer F.Cu) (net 18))
 (segment (start 92.3925 75.175) (end 93.1 75.175) (width 0.1524) (layer F.Cu) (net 18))
 (segment (start 93.345 74.93) (end 94.375 74.93) (width 0.1524) (layer F.Cu) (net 18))
 (segment (start 93.1 75.175) (end 93.345 74.93) (width 0.1524) (layer F.Cu) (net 18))
 (segment (start 118.99 75.8825) (end 119.9425 74.93) (width 0.1524) (layer F.Cu) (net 15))
 (segment (start 115.57 75.8825) (end 118.99 75.8825) (width 0.1524) (layer F.Cu) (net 15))
 (segment (start 114.035 75.565) (end 115.2525 75.565) (width 0.1524) (layer F.Cu) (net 15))
 (segment (start 115.2525 75.565) (end 115.57 75.8825) (width 0.1524) (layer F.Cu) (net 15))
 (segment (start 119.235 76.5175) (end 119.87 77.1525) (width 0.1524) (layer F.Cu) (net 16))
 (segment (start 115.57 76.5175) (end 119.235 76.5175) (width 0.1524) (layer F.Cu) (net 16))
 (segment (start 114.035 76.835) (end 115.2525 76.835) (width 0.1524) (layer F.Cu) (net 16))
 (segment (start 115.2525 76.835) (end 115.57 76.5175) (width 0.1524) (layer F.Cu) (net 16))
 (segment (start 113.9825 84.31) (end 113.9825 82.2325) (width 0.381) (layer F.Cu) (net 3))
 (segment (start 116.5875 82.2325) (end 113.9825 82.2325) (width 0.381) (layer F.Cu) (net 3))
 (segment (start 116.3625 80.025) (end 116.3775 80.01) (width 0.381) (layer F.Cu) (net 3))
 (segment (start 116.3625 82.2325) (end 116.3625 80.025) (width 0.381) (layer F.Cu) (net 3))
 (segment (start 116.5875 84.7725) (end 116.5875 83.5025) (width 0.381) (layer F.Cu) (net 2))
 (segment (start 116.3625 83.5025) (end 118.11 83.5025) (width 0.381) (layer F.Cu) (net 2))
 (segment (start 120.505 81.1075) (end 120.505 80.01) (width 0.381) (layer F.Cu) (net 2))
 (segment (start 118.11 83.5025) (end 120.505 81.1075) (width 0.381) (layer F.Cu) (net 2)))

